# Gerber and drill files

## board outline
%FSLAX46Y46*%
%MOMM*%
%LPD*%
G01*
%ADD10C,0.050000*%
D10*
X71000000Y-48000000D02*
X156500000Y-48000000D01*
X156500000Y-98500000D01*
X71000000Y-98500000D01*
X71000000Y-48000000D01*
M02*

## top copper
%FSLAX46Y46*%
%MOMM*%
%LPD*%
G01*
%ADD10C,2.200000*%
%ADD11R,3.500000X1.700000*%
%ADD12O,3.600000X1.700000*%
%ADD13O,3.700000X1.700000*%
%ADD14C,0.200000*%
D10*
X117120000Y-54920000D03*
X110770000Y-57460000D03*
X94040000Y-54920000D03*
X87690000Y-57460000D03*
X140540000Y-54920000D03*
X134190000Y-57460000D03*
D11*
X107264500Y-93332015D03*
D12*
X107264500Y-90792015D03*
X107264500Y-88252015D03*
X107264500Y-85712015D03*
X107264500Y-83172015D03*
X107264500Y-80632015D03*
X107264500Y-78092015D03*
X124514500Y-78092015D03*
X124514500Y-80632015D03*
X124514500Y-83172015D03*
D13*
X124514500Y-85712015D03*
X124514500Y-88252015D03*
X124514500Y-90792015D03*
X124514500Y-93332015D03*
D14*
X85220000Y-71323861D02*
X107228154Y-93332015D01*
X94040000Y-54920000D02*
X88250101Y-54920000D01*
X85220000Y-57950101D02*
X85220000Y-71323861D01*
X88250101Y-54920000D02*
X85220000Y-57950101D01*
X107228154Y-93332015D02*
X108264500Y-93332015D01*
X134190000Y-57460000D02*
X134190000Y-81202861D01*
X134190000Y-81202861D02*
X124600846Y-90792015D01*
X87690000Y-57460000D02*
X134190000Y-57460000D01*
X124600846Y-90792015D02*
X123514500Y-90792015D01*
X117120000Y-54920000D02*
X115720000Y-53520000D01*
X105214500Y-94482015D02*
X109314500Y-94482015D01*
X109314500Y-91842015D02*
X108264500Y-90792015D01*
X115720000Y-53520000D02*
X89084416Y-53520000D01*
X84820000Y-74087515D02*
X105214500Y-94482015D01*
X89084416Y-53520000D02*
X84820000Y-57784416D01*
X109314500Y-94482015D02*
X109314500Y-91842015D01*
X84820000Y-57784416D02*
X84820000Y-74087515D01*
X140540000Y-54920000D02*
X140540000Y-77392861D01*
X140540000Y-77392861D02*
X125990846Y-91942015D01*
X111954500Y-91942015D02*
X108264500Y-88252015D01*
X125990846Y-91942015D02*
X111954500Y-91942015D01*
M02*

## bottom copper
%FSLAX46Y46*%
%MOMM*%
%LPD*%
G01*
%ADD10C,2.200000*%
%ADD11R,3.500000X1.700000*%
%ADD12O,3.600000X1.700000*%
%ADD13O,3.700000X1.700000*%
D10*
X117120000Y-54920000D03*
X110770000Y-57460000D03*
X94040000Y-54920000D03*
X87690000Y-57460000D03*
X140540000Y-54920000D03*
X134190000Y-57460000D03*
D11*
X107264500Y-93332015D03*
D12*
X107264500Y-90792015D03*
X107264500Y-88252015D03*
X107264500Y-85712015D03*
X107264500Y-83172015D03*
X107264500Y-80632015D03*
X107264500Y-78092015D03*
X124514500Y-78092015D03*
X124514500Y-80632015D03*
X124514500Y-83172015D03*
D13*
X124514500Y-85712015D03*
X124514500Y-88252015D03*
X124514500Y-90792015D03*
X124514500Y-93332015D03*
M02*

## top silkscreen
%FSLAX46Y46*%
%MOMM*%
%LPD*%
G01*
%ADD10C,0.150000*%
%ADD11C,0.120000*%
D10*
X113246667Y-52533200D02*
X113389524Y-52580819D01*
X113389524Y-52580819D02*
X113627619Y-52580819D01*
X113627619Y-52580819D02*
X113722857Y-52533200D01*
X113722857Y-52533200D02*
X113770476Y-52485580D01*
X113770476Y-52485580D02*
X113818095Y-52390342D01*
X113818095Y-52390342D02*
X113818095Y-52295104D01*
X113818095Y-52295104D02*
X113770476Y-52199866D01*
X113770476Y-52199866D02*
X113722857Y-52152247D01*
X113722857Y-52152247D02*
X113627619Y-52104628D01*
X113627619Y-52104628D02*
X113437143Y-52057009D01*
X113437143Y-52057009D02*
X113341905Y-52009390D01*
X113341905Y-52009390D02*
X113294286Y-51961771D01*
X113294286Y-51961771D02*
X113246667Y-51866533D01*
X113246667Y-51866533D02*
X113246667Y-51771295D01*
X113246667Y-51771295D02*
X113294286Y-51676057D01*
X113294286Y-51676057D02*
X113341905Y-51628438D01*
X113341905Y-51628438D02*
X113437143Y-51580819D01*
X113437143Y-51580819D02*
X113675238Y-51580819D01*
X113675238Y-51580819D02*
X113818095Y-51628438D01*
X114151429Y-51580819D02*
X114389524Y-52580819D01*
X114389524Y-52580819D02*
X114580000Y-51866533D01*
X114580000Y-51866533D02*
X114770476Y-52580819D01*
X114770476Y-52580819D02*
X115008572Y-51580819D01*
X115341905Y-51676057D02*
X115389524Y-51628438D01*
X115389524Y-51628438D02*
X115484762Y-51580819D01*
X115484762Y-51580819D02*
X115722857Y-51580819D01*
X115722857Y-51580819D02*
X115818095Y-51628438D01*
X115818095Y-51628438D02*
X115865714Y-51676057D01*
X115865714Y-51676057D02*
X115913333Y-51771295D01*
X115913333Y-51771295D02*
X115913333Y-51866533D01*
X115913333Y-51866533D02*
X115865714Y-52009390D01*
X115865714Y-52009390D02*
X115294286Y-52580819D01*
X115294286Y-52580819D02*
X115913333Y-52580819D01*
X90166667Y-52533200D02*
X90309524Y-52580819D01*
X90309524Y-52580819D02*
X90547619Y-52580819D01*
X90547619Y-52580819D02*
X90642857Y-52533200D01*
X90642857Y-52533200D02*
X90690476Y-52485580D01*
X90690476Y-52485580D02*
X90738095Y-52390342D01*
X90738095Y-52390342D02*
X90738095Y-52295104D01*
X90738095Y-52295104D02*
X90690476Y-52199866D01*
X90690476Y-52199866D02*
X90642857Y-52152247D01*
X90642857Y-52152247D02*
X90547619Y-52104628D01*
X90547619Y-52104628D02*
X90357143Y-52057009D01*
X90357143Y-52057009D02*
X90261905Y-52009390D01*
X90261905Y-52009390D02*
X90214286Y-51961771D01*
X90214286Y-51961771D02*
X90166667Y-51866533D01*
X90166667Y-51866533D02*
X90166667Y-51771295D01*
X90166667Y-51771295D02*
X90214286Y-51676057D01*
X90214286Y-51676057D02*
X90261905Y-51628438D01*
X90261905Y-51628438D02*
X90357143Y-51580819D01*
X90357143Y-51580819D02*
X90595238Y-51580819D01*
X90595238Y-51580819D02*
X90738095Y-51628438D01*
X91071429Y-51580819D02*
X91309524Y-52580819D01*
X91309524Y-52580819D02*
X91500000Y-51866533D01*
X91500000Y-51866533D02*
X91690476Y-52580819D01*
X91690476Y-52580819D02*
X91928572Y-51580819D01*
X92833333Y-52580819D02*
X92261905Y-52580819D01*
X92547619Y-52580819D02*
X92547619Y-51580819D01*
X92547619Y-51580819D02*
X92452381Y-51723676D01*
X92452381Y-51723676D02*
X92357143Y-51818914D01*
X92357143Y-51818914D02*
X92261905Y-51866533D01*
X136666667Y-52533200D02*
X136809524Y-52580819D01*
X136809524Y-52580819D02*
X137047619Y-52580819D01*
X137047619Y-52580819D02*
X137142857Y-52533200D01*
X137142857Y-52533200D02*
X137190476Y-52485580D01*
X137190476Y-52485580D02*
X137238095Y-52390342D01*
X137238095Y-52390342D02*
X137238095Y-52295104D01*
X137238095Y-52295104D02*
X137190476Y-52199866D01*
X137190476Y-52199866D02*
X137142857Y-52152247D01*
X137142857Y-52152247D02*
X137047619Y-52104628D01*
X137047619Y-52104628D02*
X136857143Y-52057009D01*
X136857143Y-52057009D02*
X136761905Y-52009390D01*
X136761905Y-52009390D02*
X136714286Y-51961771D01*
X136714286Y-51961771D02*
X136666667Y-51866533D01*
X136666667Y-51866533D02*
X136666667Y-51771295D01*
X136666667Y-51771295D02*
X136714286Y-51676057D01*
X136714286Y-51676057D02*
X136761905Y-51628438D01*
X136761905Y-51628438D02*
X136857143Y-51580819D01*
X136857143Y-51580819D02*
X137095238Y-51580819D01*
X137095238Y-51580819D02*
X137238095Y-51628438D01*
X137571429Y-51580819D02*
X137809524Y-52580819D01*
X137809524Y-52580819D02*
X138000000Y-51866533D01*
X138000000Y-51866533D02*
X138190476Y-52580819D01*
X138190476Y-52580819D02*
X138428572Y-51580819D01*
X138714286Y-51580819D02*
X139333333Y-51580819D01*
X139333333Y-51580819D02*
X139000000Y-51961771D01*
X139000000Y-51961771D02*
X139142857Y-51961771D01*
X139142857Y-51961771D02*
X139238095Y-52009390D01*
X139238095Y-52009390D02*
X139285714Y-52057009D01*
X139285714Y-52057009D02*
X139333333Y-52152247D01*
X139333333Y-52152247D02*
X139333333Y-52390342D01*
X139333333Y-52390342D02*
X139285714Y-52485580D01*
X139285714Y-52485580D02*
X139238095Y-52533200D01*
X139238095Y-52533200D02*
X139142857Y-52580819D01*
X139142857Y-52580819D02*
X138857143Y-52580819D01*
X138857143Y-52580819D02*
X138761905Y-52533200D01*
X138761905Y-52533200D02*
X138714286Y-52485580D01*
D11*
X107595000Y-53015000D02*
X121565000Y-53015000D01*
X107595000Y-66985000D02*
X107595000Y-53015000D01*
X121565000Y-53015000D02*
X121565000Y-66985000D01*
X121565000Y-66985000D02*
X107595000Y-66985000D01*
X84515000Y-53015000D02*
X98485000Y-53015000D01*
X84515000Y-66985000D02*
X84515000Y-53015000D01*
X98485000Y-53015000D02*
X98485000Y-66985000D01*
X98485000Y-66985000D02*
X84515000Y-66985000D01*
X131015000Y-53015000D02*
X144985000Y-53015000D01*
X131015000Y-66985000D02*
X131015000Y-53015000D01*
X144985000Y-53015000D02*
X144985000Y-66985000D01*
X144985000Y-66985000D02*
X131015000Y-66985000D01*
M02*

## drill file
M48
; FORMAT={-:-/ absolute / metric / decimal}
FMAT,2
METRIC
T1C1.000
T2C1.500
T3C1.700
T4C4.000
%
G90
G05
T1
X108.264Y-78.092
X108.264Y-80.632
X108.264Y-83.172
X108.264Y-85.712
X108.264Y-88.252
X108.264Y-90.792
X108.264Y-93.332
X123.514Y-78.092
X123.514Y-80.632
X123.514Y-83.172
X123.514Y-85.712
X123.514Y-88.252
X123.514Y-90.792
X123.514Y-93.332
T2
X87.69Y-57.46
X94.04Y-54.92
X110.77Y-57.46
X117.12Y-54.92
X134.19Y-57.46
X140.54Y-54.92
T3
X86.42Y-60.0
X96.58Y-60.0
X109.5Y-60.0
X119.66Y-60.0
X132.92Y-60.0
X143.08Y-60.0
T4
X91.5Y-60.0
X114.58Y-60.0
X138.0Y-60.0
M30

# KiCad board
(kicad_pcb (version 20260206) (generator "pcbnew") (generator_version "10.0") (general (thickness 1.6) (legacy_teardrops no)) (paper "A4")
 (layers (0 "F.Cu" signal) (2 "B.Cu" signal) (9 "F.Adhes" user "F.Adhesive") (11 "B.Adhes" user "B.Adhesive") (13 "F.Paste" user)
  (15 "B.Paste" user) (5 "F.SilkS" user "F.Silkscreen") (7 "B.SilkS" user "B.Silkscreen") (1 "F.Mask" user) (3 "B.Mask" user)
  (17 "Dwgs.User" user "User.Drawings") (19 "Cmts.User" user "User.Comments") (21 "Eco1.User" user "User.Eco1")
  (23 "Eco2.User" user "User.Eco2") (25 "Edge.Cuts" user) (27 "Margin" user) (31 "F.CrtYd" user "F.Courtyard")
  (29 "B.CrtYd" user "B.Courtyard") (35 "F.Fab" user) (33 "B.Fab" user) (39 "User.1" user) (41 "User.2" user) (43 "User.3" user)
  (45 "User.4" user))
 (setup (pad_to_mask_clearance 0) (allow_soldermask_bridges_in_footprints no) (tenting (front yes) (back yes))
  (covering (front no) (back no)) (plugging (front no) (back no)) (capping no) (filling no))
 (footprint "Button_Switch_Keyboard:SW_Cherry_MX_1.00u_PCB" (layer "F.Cu") (at 117.12 54.92)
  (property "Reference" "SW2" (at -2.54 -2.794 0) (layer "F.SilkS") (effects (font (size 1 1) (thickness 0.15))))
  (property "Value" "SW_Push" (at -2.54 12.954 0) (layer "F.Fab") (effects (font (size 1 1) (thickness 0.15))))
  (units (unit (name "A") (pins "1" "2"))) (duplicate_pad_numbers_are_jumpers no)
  (fp_line (start -9.525 -1.905) (end 4.445 -1.905) (stroke (width 0.12) (type solid)) (layer "F.SilkS"))
  (fp_line (start -9.525 12.065) (end -9.525 -1.905) (stroke (width 0.12) (type solid)) (layer "F.SilkS"))
  (fp_line (start 4.445 -1.905) (end 4.445 12.065) (stroke (width 0.12) (type solid)) (layer "F.SilkS"))
  (fp_line (start 4.445 12.065) (end -9.525 12.065) (stroke (width 0.12) (type solid)) (layer "F.SilkS"))
  (pad "" np_thru_hole circle (at -7.62 5.08) (size 1.7 1.7) (drill 1.7) (layers "*.Cu" "*.Mask"))
  (pad "" np_thru_hole circle (at -2.54 5.08) (size 4 4) (drill 4) (layers "*.Cu" "*.Mask"))
  (pad "" np_thru_hole circle (at 2.54 5.08) (size 1.7 1.7) (drill 1.7) (layers "*.Cu" "*.Mask"))
  (pad "1" thru_hole circle (at 0 0) (size 2.2 2.2) (drill 1.5) (layers "*.Cu" "*.Mask") (remove_unused_layers no)
   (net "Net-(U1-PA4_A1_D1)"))
  (pad "2" thru_hole circle (at -6.35 2.54) (size 2.2 2.2) (drill 1.5) (layers "*.Cu" "*.Mask") (remove_unused_layers no) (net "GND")))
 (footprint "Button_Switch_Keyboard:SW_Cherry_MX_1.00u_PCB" (layer "F.Cu") (at 94.04 54.92)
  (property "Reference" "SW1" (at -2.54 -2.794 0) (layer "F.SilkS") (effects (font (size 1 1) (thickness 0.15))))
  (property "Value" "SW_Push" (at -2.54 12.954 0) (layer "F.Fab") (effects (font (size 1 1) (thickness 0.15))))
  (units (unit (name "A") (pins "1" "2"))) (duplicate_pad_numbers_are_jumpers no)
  (fp_line (start -9.525 -1.905) (end 4.445 -1.905) (stroke (width 0.12) (type solid)) (layer "F.SilkS"))
  (fp_line (start -9.525 12.065) (end -9.525 -1.905) (stroke (width 0.12) (type solid)) (layer "F.SilkS"))
  (fp_line (start 4.445 -1.905) (end 4.445 12.065) (stroke (width 0.12) (type solid)) (layer "F.SilkS"))
  (fp_line (start 4.445 12.065) (end -9.525 12.065) (stroke (width 0.12) (type solid)) (layer "F.SilkS"))
  (pad "" np_thru_hole circle (at -7.62 5.08) (size 1.7 1.7) (drill 1.7) (layers "*.Cu" "*.Mask"))
  (pad "" np_thru_hole circle (at -2.54 5.08) (size 4 4) (drill 4) (layers "*.Cu" "*.Mask"))
  (pad "" np_thru_hole circle (at 2.54 5.08) (size 1.7 1.7) (drill 1.7) (layers "*.Cu" "*.Mask"))
  (pad "1" thru_hole circle (at 0 0) (size 2.2 2.2) (drill 1.5) (layers "*.Cu" "*.Mask") (remove_unused_layers no)
   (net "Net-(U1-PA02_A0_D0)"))
  (pad "2" thru_hole circle (at -6.35 2.54) (size 2.2 2.2) (drill 1.5) (layers "*.Cu" "*.Mask") (remove_unused_layers no) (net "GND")))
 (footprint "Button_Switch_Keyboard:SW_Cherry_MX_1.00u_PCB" (layer "F.Cu") (at 140.54 54.92)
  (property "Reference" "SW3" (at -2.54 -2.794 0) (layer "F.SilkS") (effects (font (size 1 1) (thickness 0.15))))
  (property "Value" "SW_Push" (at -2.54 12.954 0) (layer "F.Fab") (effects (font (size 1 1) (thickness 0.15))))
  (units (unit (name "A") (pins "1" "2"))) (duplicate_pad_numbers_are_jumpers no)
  (fp_line (start -9.525 -1.905) (end 4.445 -1.905) (stroke (width 0.12) (type solid)) (layer "F.SilkS"))
  (fp_line (start -9.525 12.065) (end -9.525 -1.905) (stroke (width 0.12) (type solid)) (layer "F.SilkS"))
  (fp_line (start 4.445 -1.905) (end 4.445 12.065) (stroke (width 0.12) (type solid)) (layer "F.SilkS"))
  (fp_line (start 4.445 12.065) (end -9.525 12.065) (stroke (width 0.12) (type solid)) (layer "F.SilkS"))
  (pad "" np_thru_hole circle (at -7.62 5.08) (size 1.7 1.7) (drill 1.7) (layers "*.Cu" "*.Mask"))
  (pad "" np_thru_hole circle (at -2.54 5.08) (size 4 4) (drill 4) (layers "*.Cu" "*.Mask"))
  (pad "" np_thru_hole circle (at 2.54 5.08) (size 1.7 1.7) (drill 1.7) (layers "*.Cu" "*.Mask"))
  (pad "1" thru_hole circle (at 0 0) (size 2.2 2.2) (drill 1.5) (layers "*.Cu" "*.Mask") (remove_unused_layers no)
   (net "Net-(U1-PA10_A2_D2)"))
  (pad "2" thru_hole circle (at -6.35 2.54) (size 2.2 2.2) (drill 1.5) (layers "*.Cu" "*.Mask") (remove_unused_layers no) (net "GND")))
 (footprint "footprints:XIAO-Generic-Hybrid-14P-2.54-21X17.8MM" (layer "B.Cu") (at 115.8895 85.712015)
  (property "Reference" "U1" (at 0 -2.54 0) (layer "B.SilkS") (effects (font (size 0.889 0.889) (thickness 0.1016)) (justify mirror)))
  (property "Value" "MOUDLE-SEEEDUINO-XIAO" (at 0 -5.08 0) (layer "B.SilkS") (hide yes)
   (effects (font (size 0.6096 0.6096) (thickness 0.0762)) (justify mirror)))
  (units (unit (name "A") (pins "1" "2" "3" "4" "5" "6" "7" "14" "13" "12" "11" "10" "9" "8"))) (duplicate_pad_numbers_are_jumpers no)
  (pad "1" thru_hole rect (at -7.625 7.62) (size 3.5 1.7) (drill 1 (offset -1 0)) (layers "*.Cu" "*.Mask") (remove_unused_layers no)
   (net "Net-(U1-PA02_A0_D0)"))
  (pad "2" thru_hole oval (at -7.625 5.08) (size 3.6 1.7) (drill 1 (offset -1 0)) (layers "*.Cu" "*.Mask") (remove_unused_layers no)
   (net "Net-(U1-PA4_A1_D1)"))
  (pad "3" thru_hole oval (at -7.625 2.54) (size 3.6 1.7) (drill 1 (offset -1 0)) (layers "*.Cu" "*.Mask") (remove_unused_layers no)
   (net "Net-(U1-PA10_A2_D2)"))
  (pad "4" thru_hole oval (at -7.625 0) (size 3.6 1.7) (drill 1 (offset -1 0)) (layers "*.Cu" "*.Mask") (remove_unused_layers no)
   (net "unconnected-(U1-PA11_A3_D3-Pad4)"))
  (pad "5" thru_hole oval (at -7.625 -2.54) (size 3.6 1.7) (drill 1 (offset -1 0)) (layers "*.Cu" "*.Mask") (remove_unused_layers no)
   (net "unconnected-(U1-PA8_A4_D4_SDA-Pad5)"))
  (pad "6" thru_hole oval (at -7.625 -5.08 180) (size 3.6 1.7) (drill 1 (offset 1 0)) (layers "*.Cu" "*.Mask") (remove_unused_layers no)
   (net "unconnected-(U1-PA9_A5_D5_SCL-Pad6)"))
  (pad "7" thru_hole oval (at -7.625 -7.62) (size 3.6 1.7) (drill 1 (offset -1 0)) (layers "*.Cu" "*.Mask") (remove_unused_layers no)
   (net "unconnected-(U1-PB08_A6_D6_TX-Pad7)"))
  (pad "8" thru_hole oval (at 7.625 -7.62) (size 3.6 1.7) (drill 1 (offset 1 0)) (layers "*.Cu" "*.Mask") (remove_unused_layers no)
   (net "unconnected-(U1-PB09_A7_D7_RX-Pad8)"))
  (pad "9" thru_hole oval (at 7.625 -5.08) (size 3.6 1.7) (drill 1 (offset 1 0)) (layers "*.Cu" "*.Mask") (remove_unused_layers no)
   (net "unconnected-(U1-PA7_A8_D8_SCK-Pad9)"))
  (pad "10" thru_hole oval (at 7.625 -2.54) (size 3.6 1.7) (drill 1 (offset 1 0)) (layers "*.Cu" "*.Mask") (remove_unused_layers no)
   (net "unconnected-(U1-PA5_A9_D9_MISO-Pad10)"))
  (pad "11" thru_hole oval (at 7.625 0) (size 3.7 1.7) (drill 1 (offset 1 0)) (layers "*.Cu" "*.Mask") (remove_unused_layers no)
   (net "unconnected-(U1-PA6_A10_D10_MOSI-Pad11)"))
  (pad "12" thru_hole oval (at 7.625 2.54) (size 3.7 1.7) (drill 1 (offset 1 0)) (layers "*.Cu" "*.Mask") (remove_unused_layers no)
   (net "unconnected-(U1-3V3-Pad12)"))
  (pad "13" thru_hole oval (at 7.625 5.08) (size 3.7 1.7) (drill 1 (offset 1 0)) (layers "*.Cu" "*.Mask") (remove_unused_layers no)
   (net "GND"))
  (pad "14" thru_hole oval (at 7.625 7.62) (size 3.7 1.7) (drill 1 (offset 1 0)) (layers "*.Cu" "*.Mask") (remove_unused_layers no)
   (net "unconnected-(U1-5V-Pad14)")))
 (gr_rect (start 71 48) (end 156.5 98.5) (stroke (width 0.05) (type default)) (fill no) (layer "Edge.Cuts"))
 (segment (start 85.22 71.323861) (end 107.228154 93.332015) (width 0.2) (layer "F.Cu") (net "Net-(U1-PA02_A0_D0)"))
 (segment (start 94.04 54.92) (end 88.250101 54.92) (width 0.2) (layer "F.Cu") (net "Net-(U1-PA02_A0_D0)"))
 (segment (start 85.22 57.950101) (end 85.22 71.323861) (width 0.2) (layer "F.Cu") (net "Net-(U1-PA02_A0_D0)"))
 (segment (start 88.250101 54.92) (end 85.22 57.950101) (width 0.2) (layer "F.Cu") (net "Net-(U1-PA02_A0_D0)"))
 (segment (start 107.228154 93.332015) (end 108.2645 93.332015) (width 0.2) (layer "F.Cu") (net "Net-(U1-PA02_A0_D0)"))
 (segment (start 134.19 57.46) (end 134.19 81.202861) (width 0.2) (layer "F.Cu") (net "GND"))
 (segment (start 134.19 81.202861) (end 124.600846 90.792015) (width 0.2) (layer "F.Cu") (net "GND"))
 (segment (start 87.69 57.46) (end 134.19 57.46) (width 0.2) (layer "F.Cu") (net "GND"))
 (segment (start 124.600846 90.792015) (end 123.5145 90.792015) (width 0.2) (layer "F.Cu") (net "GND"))
 (segment (start 117.12 54.92) (end 115.72 53.52) (width 0.2) (layer "F.Cu") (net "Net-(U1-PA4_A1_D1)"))
 (segment (start 105.2145 94.482015) (end 109.3145 94.482015) (width 0.2) (layer "F.Cu") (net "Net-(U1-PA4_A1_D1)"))
 (segment (start 109.3145 91.842015) (end 108.2645 90.792015) (width 0.2) (layer "F.Cu") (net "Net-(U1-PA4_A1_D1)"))
 (segment (start 115.72 53.52) (end 89.084416 53.52) (width 0.2) (layer "F.Cu") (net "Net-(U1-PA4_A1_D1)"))
 (segment (start 84.82 74.087515) (end 105.2145 94.482015) (width 0.2) (layer "F.Cu") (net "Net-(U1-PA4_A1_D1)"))
 (segment (start 89.084416 53.52) (end 84.82 57.784416) (width 0.2) (layer "F.Cu") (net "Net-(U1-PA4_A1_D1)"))
 (segment (start 109.3145 94.482015) (end 109.3145 91.842015) (width 0.2) (layer "F.Cu") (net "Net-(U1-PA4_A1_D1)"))
 (segment (start 84.82 57.784416) (end 84.82 74.087515) (width 0.2) (layer "F.Cu") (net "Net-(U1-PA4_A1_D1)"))
 (segment (start 140.54 54.92) (end 140.54 77.392861) (width 0.2) (layer "F.Cu") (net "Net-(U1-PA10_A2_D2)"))
 (segment (start 140.54 77.392861) (end 125.990846 91.942015) (width 0.2) (layer "F.Cu") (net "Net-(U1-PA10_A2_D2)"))
 (segment (start 111.9545 91.942015) (end 108.2645 88.252015) (width 0.2) (layer "F.Cu") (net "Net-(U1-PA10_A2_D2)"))
 (segment (start 125.990846 91.942015) (end 111.9545 91.942015) (width 0.2) (layer "F.Cu") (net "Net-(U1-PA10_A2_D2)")))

